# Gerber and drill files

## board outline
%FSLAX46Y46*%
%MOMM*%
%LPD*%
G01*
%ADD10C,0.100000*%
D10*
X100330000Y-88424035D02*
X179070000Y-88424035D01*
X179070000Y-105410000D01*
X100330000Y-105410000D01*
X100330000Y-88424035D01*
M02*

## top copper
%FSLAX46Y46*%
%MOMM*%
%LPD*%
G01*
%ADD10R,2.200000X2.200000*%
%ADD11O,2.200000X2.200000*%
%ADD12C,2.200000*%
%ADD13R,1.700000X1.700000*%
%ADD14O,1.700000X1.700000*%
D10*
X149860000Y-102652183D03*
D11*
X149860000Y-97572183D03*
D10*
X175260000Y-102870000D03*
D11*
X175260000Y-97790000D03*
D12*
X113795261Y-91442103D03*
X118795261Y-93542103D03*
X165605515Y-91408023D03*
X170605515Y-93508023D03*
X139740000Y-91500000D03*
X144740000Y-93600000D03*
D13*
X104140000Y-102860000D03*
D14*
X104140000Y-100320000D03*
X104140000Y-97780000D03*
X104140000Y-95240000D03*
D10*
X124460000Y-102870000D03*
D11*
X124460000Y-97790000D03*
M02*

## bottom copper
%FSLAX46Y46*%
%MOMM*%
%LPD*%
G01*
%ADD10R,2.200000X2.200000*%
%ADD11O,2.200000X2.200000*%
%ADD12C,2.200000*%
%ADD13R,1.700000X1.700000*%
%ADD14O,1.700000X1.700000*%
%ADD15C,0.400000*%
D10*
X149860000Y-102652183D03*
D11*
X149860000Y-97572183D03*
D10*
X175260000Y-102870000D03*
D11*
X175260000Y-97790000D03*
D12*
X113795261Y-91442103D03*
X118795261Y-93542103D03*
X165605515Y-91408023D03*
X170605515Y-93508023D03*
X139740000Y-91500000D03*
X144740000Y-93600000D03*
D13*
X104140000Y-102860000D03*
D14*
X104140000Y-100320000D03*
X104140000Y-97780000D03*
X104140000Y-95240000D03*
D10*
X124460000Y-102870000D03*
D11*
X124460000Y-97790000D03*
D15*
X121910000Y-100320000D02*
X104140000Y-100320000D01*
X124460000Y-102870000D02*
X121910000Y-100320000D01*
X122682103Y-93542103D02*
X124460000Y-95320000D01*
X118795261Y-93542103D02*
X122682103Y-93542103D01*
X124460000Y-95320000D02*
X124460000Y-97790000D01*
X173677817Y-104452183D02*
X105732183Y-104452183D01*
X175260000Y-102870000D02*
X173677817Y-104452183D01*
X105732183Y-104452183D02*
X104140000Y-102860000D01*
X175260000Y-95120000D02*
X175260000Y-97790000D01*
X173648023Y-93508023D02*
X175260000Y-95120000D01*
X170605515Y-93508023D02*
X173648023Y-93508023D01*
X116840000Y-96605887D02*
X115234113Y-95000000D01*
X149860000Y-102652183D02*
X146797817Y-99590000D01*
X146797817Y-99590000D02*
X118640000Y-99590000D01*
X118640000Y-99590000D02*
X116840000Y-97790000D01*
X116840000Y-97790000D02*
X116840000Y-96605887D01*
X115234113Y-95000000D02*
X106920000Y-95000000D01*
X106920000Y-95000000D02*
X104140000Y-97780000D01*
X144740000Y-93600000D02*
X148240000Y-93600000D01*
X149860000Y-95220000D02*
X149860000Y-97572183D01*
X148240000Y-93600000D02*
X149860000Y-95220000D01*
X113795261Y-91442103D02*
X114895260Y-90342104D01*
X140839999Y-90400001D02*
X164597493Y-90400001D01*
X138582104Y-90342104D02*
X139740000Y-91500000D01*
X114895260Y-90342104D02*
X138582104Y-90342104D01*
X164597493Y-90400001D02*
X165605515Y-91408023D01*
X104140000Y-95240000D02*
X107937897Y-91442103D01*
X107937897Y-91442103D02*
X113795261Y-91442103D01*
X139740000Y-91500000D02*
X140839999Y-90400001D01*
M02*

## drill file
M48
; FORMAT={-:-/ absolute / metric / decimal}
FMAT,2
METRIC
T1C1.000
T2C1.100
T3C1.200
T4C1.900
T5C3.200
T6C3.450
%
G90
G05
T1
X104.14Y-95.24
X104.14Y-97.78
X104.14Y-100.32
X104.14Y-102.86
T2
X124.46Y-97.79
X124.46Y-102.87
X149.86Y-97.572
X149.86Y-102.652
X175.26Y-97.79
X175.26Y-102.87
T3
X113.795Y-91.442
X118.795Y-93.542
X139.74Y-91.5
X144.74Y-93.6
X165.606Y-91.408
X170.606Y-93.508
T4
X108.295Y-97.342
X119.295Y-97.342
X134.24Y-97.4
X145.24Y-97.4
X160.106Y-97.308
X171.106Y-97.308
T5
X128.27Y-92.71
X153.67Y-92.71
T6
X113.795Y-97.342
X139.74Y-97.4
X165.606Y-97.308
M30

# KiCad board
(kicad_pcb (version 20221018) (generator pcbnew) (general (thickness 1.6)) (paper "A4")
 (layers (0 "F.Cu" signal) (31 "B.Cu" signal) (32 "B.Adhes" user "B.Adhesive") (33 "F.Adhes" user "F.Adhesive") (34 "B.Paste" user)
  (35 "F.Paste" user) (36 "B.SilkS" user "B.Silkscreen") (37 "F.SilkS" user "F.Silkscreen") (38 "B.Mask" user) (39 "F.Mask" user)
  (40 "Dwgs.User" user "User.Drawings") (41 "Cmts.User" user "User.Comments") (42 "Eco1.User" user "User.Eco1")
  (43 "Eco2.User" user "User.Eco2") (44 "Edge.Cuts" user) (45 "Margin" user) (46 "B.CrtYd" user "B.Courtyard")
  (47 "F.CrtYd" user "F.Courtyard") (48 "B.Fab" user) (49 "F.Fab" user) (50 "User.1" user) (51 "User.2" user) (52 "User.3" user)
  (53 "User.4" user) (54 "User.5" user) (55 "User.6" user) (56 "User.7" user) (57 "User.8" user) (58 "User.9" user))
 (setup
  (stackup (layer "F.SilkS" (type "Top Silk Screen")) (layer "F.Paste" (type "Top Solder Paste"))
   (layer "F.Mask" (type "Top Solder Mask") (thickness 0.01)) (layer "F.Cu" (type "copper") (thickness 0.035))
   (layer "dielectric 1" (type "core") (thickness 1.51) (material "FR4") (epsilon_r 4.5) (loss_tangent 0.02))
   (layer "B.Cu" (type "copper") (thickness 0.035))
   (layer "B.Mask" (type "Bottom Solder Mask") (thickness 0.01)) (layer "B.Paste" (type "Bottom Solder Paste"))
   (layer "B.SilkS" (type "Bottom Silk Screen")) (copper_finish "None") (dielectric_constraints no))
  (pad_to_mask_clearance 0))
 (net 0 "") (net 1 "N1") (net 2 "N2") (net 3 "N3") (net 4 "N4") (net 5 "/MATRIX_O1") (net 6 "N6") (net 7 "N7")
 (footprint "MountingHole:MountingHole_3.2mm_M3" (layer "F.Cu") (at 128.27 92.71)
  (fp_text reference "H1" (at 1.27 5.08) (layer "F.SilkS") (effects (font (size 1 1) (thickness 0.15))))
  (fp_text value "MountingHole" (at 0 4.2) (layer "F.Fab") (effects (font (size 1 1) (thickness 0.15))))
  (pad "" np_thru_hole circle (at 0 0) (size 3.2 3.2) (drill 3.2) (layers "*.Cu" "*.Mask")))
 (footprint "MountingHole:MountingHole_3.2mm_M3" (layer "F.Cu") (at 153.67 92.71)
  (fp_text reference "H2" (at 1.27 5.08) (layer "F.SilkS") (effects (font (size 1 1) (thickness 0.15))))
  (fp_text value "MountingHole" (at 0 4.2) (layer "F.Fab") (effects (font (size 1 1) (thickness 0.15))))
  (pad "" np_thru_hole circle (at 0 0) (size 3.2 3.2) (drill 3.2) (layers "*.Cu" "*.Mask")))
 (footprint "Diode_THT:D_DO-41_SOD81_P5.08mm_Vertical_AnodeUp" (layer "F.Cu") (at 149.86 102.652183 90)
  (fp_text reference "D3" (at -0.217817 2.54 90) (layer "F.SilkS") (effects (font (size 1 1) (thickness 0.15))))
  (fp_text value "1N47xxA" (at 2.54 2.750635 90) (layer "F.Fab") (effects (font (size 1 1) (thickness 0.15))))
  (pad "1" thru_hole rect (at 0 0 90) (size 2.2 2.2) (drill 1.1) (layers "*.Cu" "*.Mask") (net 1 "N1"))
  (pad "2" thru_hole oval (at 5.08 0 90) (size 2.2 2.2) (drill 1.1) (layers "*.Cu" "*.Mask") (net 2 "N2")))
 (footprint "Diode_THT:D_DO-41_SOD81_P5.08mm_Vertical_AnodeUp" (layer "F.Cu") (at 175.26 102.87 90)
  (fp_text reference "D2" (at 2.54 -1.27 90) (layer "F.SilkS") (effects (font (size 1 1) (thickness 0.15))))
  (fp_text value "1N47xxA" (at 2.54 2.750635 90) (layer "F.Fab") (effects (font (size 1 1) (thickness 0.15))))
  (pad "1" thru_hole rect (at 0 0 90) (size 2.2 2.2) (drill 1.1) (layers "*.Cu" "*.Mask") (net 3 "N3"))
  (pad "2" thru_hole oval (at 5.08 0 90) (size 2.2 2.2) (drill 1.1) (layers "*.Cu" "*.Mask") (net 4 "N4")))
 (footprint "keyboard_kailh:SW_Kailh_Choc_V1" (layer "F.Cu") (at 113.795261 97.342103)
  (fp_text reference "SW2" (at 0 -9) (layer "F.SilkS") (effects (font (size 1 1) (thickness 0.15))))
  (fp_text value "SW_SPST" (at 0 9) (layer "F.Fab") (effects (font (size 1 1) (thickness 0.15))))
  (pad "" np_thru_hole circle (at -5.5 0) (size 1.9 1.9) (drill 1.9) (layers "*.Cu" "*.Mask"))
  (pad "" smd circle (at 0 -5.9) (size 1.25 1.25) (layers "F.Mask"))
  (pad "" np_thru_hole circle (at 0 0) (size 3.45 3.45) (drill 3.45) (layers "*.Cu" "*.Mask"))
  (pad "" smd circle (at 5 -3.8) (size 1.25 1.25) (layers "F.Mask"))
  (pad "" np_thru_hole circle (at 5.5 0) (size 1.9 1.9) (drill 1.9) (layers "*.Cu" "*.Mask"))
  (pad "1" thru_hole circle (at 0 -5.9) (size 2.2 2.2) (drill 1.2) (layers "*.Cu" "B.Mask") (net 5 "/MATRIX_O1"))
  (pad "2" thru_hole circle (at 5 -3.8) (size 2.2 2.2) (drill 1.2) (layers "*.Cu" "B.Mask") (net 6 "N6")))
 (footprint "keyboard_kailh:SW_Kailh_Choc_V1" (layer "F.Cu") (at 165.605515 97.308023)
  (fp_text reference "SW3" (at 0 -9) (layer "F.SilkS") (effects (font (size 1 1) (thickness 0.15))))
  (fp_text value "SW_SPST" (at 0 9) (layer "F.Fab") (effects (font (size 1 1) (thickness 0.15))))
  (pad "" np_thru_hole circle (at -5.5 0) (size 1.9 1.9) (drill 1.9) (layers "*.Cu" "*.Mask"))
  (pad "" smd circle (at 0 -5.9) (size 1.25 1.25) (layers "F.Mask"))
  (pad "" np_thru_hole circle (at 0 0) (size 3.45 3.45) (drill 3.45) (layers "*.Cu" "*.Mask"))
  (pad "" smd circle (at 5 -3.8) (size 1.25 1.25) (layers "F.Mask"))
  (pad "" np_thru_hole circle (at 5.5 0) (size 1.9 1.9) (drill 1.9) (layers "*.Cu" "*.Mask"))
  (pad "1" thru_hole circle (at 0 -5.9) (size 2.2 2.2) (drill 1.2) (layers "*.Cu" "B.Mask") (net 5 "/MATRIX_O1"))
  (pad "2" thru_hole circle (at 5 -3.8) (size 2.2 2.2) (drill 1.2) (layers "*.Cu" "B.Mask") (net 4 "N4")))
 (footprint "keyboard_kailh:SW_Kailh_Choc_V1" (layer "F.Cu") (at 139.74 97.4)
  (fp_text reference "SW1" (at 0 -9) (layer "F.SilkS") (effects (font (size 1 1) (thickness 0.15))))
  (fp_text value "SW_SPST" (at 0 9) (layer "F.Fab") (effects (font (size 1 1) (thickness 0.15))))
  (pad "" np_thru_hole circle (at -5.5 0) (size 1.9 1.9) (drill 1.9) (layers "*.Cu" "*.Mask"))
  (pad "" smd circle (at 0 -5.9) (size 1.25 1.25) (layers "F.Mask"))
  (pad "" np_thru_hole circle (at 0 0) (size 3.45 3.45) (drill 3.45) (layers "*.Cu" "*.Mask"))
  (pad "" smd circle (at 5 -3.8) (size 1.25 1.25) (layers "F.Mask"))
  (pad "" np_thru_hole circle (at 5.5 0) (size 1.9 1.9) (drill 1.9) (layers "*.Cu" "*.Mask"))
  (pad "1" thru_hole circle (at 0 -5.9) (size 2.2 2.2) (drill 1.2) (layers "*.Cu" "B.Mask") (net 5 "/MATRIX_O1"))
  (pad "2" thru_hole circle (at 5 -3.8) (size 2.2 2.2) (drill 1.2) (layers "*.Cu" "B.Mask") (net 2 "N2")))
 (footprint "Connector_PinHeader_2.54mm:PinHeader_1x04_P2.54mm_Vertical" (layer "F.Cu") (at 104.14 102.86 180)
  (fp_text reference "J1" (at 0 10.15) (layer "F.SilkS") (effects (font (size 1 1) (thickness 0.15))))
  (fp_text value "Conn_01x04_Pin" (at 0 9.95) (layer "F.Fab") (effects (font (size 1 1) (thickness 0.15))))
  (pad "1" thru_hole rect (at 0 0 180) (size 1.7 1.7) (drill 1) (layers "*.Cu" "*.Mask") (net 3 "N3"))
  (pad "2" thru_hole oval (at 0 2.54 180) (size 1.7 1.7) (drill 1) (layers "*.Cu" "*.Mask") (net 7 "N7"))
  (pad "3" thru_hole oval (at 0 5.08 180) (size 1.7 1.7) (drill 1) (layers "*.Cu" "*.Mask") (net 1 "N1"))
  (pad "4" thru_hole oval (at 0 7.62 180) (size 1.7 1.7) (drill 1) (layers "*.Cu" "*.Mask") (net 5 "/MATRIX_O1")))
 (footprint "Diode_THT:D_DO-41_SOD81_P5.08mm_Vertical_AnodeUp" (layer "F.Cu") (at 124.46 102.87 90)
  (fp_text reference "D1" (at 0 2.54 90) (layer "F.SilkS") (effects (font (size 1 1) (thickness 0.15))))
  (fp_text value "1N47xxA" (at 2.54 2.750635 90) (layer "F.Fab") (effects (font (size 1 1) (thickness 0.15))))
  (pad "1" thru_hole rect (at 0 0 90) (size 2.2 2.2) (drill 1.1) (layers "*.Cu" "*.Mask") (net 7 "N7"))
  (pad "2" thru_hole oval (at 5.08 0 90) (size 2.2 2.2) (drill 1.1) (layers "*.Cu" "*.Mask") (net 6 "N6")))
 (gr_rect (start 100.33 88.424035) (end 179.07 105.41) (stroke (width 0.1) (type default)) (fill none) (layer "Edge.Cuts"))
 (segment (start 121.91 100.32) (end 104.14 100.32) (width 0.4) (layer "B.Cu") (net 7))
 (segment (start 124.46 102.87) (end 121.91 100.32) (width 0.4) (layer "B.Cu") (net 7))
 (segment (start 122.682103 93.542103) (end 124.46 95.32) (width 0.4) (layer "B.Cu") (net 6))
 (segment (start 118.795261 93.542103) (end 122.682103 93.542103) (width 0.4) (layer "B.Cu") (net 6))
 (segment (start 124.46 95.32) (end 124.46 97.79) (width 0.4) (layer "B.Cu") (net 6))
 (segment (start 173.677817 104.452183) (end 105.732183 104.452183) (width 0.4) (layer "B.Cu") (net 3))
 (segment (start 175.26 102.87) (end 173.677817 104.452183) (width 0.4) (layer "B.Cu") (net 3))
 (segment (start 105.732183 104.452183) (end 104.14 102.86) (width 0.4) (layer "B.Cu") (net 3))
 (segment (start 175.26 95.12) (end 175.26 97.79) (width 0.4) (layer "B.Cu") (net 4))
 (segment (start 173.648023 93.508023) (end 175.26 95.12) (width 0.4) (layer "B.Cu") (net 4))
 (segment (start 170.605515 93.508023) (end 173.648023 93.508023) (width 0.4) (layer "B.Cu") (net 4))
 (segment (start 116.84 96.605887) (end 115.234113 95) (width 0.4) (layer "B.Cu") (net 1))
 (segment (start 149.86 102.652183) (end 146.797817 99.59) (width 0.4) (layer "B.Cu") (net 1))
 (segment (start 146.797817 99.59) (end 118.64 99.59) (width 0.4) (layer "B.Cu") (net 1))
 (segment (start 118.64 99.59) (end 116.84 97.79) (width 0.4) (layer "B.Cu") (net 1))
 (segment (start 116.84 97.79) (end 116.84 96.605887) (width 0.4) (layer "B.Cu") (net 1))
 (segment (start 115.234113 95) (end 106.92 95) (width 0.4) (layer "B.Cu") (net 1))
 (segment (start 106.92 95) (end 104.14 97.78) (width 0.4) (layer "B.Cu") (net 1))
 (segment (start 144.74 93.6) (end 148.24 93.6) (width 0.4) (layer "B.Cu") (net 2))
 (segment (start 149.86 95.22) (end 149.86 97.572183) (width 0.4) (layer "B.Cu") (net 2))
 (segment (start 148.24 93.6) (end 149.86 95.22) (width 0.4) (layer "B.Cu") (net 2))
 (segment (start 113.795261 91.442103) (end 114.89526 90.342104) (width 0.4) (layer "B.Cu") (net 5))
 (segment (start 140.839999 90.400001) (end 164.597493 90.400001) (width 0.4) (layer "B.Cu") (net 5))
 (segment (start 138.582104 90.342104) (end 139.74 91.5) (width 0.4) (layer "B.Cu") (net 5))
 (segment (start 114.89526 90.342104) (end 138.582104 90.342104) (width 0.4) (layer "B.Cu") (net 5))
 (segment (start 164.597493 90.400001) (end 165.605515 91.408023) (width 0.4) (layer "B.Cu") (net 5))
 (segment (start 104.14 95.24) (end 107.937897 91.442103) (width 0.4) (layer "B.Cu") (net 5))
 (segment (start 107.937897 91.442103) (end 113.795261 91.442103) (width 0.4) (layer "B.Cu") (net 5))
 (segment (start 139.74 91.5) (end 140.839999 90.400001) (width 0.4) (layer "B.Cu") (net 5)))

